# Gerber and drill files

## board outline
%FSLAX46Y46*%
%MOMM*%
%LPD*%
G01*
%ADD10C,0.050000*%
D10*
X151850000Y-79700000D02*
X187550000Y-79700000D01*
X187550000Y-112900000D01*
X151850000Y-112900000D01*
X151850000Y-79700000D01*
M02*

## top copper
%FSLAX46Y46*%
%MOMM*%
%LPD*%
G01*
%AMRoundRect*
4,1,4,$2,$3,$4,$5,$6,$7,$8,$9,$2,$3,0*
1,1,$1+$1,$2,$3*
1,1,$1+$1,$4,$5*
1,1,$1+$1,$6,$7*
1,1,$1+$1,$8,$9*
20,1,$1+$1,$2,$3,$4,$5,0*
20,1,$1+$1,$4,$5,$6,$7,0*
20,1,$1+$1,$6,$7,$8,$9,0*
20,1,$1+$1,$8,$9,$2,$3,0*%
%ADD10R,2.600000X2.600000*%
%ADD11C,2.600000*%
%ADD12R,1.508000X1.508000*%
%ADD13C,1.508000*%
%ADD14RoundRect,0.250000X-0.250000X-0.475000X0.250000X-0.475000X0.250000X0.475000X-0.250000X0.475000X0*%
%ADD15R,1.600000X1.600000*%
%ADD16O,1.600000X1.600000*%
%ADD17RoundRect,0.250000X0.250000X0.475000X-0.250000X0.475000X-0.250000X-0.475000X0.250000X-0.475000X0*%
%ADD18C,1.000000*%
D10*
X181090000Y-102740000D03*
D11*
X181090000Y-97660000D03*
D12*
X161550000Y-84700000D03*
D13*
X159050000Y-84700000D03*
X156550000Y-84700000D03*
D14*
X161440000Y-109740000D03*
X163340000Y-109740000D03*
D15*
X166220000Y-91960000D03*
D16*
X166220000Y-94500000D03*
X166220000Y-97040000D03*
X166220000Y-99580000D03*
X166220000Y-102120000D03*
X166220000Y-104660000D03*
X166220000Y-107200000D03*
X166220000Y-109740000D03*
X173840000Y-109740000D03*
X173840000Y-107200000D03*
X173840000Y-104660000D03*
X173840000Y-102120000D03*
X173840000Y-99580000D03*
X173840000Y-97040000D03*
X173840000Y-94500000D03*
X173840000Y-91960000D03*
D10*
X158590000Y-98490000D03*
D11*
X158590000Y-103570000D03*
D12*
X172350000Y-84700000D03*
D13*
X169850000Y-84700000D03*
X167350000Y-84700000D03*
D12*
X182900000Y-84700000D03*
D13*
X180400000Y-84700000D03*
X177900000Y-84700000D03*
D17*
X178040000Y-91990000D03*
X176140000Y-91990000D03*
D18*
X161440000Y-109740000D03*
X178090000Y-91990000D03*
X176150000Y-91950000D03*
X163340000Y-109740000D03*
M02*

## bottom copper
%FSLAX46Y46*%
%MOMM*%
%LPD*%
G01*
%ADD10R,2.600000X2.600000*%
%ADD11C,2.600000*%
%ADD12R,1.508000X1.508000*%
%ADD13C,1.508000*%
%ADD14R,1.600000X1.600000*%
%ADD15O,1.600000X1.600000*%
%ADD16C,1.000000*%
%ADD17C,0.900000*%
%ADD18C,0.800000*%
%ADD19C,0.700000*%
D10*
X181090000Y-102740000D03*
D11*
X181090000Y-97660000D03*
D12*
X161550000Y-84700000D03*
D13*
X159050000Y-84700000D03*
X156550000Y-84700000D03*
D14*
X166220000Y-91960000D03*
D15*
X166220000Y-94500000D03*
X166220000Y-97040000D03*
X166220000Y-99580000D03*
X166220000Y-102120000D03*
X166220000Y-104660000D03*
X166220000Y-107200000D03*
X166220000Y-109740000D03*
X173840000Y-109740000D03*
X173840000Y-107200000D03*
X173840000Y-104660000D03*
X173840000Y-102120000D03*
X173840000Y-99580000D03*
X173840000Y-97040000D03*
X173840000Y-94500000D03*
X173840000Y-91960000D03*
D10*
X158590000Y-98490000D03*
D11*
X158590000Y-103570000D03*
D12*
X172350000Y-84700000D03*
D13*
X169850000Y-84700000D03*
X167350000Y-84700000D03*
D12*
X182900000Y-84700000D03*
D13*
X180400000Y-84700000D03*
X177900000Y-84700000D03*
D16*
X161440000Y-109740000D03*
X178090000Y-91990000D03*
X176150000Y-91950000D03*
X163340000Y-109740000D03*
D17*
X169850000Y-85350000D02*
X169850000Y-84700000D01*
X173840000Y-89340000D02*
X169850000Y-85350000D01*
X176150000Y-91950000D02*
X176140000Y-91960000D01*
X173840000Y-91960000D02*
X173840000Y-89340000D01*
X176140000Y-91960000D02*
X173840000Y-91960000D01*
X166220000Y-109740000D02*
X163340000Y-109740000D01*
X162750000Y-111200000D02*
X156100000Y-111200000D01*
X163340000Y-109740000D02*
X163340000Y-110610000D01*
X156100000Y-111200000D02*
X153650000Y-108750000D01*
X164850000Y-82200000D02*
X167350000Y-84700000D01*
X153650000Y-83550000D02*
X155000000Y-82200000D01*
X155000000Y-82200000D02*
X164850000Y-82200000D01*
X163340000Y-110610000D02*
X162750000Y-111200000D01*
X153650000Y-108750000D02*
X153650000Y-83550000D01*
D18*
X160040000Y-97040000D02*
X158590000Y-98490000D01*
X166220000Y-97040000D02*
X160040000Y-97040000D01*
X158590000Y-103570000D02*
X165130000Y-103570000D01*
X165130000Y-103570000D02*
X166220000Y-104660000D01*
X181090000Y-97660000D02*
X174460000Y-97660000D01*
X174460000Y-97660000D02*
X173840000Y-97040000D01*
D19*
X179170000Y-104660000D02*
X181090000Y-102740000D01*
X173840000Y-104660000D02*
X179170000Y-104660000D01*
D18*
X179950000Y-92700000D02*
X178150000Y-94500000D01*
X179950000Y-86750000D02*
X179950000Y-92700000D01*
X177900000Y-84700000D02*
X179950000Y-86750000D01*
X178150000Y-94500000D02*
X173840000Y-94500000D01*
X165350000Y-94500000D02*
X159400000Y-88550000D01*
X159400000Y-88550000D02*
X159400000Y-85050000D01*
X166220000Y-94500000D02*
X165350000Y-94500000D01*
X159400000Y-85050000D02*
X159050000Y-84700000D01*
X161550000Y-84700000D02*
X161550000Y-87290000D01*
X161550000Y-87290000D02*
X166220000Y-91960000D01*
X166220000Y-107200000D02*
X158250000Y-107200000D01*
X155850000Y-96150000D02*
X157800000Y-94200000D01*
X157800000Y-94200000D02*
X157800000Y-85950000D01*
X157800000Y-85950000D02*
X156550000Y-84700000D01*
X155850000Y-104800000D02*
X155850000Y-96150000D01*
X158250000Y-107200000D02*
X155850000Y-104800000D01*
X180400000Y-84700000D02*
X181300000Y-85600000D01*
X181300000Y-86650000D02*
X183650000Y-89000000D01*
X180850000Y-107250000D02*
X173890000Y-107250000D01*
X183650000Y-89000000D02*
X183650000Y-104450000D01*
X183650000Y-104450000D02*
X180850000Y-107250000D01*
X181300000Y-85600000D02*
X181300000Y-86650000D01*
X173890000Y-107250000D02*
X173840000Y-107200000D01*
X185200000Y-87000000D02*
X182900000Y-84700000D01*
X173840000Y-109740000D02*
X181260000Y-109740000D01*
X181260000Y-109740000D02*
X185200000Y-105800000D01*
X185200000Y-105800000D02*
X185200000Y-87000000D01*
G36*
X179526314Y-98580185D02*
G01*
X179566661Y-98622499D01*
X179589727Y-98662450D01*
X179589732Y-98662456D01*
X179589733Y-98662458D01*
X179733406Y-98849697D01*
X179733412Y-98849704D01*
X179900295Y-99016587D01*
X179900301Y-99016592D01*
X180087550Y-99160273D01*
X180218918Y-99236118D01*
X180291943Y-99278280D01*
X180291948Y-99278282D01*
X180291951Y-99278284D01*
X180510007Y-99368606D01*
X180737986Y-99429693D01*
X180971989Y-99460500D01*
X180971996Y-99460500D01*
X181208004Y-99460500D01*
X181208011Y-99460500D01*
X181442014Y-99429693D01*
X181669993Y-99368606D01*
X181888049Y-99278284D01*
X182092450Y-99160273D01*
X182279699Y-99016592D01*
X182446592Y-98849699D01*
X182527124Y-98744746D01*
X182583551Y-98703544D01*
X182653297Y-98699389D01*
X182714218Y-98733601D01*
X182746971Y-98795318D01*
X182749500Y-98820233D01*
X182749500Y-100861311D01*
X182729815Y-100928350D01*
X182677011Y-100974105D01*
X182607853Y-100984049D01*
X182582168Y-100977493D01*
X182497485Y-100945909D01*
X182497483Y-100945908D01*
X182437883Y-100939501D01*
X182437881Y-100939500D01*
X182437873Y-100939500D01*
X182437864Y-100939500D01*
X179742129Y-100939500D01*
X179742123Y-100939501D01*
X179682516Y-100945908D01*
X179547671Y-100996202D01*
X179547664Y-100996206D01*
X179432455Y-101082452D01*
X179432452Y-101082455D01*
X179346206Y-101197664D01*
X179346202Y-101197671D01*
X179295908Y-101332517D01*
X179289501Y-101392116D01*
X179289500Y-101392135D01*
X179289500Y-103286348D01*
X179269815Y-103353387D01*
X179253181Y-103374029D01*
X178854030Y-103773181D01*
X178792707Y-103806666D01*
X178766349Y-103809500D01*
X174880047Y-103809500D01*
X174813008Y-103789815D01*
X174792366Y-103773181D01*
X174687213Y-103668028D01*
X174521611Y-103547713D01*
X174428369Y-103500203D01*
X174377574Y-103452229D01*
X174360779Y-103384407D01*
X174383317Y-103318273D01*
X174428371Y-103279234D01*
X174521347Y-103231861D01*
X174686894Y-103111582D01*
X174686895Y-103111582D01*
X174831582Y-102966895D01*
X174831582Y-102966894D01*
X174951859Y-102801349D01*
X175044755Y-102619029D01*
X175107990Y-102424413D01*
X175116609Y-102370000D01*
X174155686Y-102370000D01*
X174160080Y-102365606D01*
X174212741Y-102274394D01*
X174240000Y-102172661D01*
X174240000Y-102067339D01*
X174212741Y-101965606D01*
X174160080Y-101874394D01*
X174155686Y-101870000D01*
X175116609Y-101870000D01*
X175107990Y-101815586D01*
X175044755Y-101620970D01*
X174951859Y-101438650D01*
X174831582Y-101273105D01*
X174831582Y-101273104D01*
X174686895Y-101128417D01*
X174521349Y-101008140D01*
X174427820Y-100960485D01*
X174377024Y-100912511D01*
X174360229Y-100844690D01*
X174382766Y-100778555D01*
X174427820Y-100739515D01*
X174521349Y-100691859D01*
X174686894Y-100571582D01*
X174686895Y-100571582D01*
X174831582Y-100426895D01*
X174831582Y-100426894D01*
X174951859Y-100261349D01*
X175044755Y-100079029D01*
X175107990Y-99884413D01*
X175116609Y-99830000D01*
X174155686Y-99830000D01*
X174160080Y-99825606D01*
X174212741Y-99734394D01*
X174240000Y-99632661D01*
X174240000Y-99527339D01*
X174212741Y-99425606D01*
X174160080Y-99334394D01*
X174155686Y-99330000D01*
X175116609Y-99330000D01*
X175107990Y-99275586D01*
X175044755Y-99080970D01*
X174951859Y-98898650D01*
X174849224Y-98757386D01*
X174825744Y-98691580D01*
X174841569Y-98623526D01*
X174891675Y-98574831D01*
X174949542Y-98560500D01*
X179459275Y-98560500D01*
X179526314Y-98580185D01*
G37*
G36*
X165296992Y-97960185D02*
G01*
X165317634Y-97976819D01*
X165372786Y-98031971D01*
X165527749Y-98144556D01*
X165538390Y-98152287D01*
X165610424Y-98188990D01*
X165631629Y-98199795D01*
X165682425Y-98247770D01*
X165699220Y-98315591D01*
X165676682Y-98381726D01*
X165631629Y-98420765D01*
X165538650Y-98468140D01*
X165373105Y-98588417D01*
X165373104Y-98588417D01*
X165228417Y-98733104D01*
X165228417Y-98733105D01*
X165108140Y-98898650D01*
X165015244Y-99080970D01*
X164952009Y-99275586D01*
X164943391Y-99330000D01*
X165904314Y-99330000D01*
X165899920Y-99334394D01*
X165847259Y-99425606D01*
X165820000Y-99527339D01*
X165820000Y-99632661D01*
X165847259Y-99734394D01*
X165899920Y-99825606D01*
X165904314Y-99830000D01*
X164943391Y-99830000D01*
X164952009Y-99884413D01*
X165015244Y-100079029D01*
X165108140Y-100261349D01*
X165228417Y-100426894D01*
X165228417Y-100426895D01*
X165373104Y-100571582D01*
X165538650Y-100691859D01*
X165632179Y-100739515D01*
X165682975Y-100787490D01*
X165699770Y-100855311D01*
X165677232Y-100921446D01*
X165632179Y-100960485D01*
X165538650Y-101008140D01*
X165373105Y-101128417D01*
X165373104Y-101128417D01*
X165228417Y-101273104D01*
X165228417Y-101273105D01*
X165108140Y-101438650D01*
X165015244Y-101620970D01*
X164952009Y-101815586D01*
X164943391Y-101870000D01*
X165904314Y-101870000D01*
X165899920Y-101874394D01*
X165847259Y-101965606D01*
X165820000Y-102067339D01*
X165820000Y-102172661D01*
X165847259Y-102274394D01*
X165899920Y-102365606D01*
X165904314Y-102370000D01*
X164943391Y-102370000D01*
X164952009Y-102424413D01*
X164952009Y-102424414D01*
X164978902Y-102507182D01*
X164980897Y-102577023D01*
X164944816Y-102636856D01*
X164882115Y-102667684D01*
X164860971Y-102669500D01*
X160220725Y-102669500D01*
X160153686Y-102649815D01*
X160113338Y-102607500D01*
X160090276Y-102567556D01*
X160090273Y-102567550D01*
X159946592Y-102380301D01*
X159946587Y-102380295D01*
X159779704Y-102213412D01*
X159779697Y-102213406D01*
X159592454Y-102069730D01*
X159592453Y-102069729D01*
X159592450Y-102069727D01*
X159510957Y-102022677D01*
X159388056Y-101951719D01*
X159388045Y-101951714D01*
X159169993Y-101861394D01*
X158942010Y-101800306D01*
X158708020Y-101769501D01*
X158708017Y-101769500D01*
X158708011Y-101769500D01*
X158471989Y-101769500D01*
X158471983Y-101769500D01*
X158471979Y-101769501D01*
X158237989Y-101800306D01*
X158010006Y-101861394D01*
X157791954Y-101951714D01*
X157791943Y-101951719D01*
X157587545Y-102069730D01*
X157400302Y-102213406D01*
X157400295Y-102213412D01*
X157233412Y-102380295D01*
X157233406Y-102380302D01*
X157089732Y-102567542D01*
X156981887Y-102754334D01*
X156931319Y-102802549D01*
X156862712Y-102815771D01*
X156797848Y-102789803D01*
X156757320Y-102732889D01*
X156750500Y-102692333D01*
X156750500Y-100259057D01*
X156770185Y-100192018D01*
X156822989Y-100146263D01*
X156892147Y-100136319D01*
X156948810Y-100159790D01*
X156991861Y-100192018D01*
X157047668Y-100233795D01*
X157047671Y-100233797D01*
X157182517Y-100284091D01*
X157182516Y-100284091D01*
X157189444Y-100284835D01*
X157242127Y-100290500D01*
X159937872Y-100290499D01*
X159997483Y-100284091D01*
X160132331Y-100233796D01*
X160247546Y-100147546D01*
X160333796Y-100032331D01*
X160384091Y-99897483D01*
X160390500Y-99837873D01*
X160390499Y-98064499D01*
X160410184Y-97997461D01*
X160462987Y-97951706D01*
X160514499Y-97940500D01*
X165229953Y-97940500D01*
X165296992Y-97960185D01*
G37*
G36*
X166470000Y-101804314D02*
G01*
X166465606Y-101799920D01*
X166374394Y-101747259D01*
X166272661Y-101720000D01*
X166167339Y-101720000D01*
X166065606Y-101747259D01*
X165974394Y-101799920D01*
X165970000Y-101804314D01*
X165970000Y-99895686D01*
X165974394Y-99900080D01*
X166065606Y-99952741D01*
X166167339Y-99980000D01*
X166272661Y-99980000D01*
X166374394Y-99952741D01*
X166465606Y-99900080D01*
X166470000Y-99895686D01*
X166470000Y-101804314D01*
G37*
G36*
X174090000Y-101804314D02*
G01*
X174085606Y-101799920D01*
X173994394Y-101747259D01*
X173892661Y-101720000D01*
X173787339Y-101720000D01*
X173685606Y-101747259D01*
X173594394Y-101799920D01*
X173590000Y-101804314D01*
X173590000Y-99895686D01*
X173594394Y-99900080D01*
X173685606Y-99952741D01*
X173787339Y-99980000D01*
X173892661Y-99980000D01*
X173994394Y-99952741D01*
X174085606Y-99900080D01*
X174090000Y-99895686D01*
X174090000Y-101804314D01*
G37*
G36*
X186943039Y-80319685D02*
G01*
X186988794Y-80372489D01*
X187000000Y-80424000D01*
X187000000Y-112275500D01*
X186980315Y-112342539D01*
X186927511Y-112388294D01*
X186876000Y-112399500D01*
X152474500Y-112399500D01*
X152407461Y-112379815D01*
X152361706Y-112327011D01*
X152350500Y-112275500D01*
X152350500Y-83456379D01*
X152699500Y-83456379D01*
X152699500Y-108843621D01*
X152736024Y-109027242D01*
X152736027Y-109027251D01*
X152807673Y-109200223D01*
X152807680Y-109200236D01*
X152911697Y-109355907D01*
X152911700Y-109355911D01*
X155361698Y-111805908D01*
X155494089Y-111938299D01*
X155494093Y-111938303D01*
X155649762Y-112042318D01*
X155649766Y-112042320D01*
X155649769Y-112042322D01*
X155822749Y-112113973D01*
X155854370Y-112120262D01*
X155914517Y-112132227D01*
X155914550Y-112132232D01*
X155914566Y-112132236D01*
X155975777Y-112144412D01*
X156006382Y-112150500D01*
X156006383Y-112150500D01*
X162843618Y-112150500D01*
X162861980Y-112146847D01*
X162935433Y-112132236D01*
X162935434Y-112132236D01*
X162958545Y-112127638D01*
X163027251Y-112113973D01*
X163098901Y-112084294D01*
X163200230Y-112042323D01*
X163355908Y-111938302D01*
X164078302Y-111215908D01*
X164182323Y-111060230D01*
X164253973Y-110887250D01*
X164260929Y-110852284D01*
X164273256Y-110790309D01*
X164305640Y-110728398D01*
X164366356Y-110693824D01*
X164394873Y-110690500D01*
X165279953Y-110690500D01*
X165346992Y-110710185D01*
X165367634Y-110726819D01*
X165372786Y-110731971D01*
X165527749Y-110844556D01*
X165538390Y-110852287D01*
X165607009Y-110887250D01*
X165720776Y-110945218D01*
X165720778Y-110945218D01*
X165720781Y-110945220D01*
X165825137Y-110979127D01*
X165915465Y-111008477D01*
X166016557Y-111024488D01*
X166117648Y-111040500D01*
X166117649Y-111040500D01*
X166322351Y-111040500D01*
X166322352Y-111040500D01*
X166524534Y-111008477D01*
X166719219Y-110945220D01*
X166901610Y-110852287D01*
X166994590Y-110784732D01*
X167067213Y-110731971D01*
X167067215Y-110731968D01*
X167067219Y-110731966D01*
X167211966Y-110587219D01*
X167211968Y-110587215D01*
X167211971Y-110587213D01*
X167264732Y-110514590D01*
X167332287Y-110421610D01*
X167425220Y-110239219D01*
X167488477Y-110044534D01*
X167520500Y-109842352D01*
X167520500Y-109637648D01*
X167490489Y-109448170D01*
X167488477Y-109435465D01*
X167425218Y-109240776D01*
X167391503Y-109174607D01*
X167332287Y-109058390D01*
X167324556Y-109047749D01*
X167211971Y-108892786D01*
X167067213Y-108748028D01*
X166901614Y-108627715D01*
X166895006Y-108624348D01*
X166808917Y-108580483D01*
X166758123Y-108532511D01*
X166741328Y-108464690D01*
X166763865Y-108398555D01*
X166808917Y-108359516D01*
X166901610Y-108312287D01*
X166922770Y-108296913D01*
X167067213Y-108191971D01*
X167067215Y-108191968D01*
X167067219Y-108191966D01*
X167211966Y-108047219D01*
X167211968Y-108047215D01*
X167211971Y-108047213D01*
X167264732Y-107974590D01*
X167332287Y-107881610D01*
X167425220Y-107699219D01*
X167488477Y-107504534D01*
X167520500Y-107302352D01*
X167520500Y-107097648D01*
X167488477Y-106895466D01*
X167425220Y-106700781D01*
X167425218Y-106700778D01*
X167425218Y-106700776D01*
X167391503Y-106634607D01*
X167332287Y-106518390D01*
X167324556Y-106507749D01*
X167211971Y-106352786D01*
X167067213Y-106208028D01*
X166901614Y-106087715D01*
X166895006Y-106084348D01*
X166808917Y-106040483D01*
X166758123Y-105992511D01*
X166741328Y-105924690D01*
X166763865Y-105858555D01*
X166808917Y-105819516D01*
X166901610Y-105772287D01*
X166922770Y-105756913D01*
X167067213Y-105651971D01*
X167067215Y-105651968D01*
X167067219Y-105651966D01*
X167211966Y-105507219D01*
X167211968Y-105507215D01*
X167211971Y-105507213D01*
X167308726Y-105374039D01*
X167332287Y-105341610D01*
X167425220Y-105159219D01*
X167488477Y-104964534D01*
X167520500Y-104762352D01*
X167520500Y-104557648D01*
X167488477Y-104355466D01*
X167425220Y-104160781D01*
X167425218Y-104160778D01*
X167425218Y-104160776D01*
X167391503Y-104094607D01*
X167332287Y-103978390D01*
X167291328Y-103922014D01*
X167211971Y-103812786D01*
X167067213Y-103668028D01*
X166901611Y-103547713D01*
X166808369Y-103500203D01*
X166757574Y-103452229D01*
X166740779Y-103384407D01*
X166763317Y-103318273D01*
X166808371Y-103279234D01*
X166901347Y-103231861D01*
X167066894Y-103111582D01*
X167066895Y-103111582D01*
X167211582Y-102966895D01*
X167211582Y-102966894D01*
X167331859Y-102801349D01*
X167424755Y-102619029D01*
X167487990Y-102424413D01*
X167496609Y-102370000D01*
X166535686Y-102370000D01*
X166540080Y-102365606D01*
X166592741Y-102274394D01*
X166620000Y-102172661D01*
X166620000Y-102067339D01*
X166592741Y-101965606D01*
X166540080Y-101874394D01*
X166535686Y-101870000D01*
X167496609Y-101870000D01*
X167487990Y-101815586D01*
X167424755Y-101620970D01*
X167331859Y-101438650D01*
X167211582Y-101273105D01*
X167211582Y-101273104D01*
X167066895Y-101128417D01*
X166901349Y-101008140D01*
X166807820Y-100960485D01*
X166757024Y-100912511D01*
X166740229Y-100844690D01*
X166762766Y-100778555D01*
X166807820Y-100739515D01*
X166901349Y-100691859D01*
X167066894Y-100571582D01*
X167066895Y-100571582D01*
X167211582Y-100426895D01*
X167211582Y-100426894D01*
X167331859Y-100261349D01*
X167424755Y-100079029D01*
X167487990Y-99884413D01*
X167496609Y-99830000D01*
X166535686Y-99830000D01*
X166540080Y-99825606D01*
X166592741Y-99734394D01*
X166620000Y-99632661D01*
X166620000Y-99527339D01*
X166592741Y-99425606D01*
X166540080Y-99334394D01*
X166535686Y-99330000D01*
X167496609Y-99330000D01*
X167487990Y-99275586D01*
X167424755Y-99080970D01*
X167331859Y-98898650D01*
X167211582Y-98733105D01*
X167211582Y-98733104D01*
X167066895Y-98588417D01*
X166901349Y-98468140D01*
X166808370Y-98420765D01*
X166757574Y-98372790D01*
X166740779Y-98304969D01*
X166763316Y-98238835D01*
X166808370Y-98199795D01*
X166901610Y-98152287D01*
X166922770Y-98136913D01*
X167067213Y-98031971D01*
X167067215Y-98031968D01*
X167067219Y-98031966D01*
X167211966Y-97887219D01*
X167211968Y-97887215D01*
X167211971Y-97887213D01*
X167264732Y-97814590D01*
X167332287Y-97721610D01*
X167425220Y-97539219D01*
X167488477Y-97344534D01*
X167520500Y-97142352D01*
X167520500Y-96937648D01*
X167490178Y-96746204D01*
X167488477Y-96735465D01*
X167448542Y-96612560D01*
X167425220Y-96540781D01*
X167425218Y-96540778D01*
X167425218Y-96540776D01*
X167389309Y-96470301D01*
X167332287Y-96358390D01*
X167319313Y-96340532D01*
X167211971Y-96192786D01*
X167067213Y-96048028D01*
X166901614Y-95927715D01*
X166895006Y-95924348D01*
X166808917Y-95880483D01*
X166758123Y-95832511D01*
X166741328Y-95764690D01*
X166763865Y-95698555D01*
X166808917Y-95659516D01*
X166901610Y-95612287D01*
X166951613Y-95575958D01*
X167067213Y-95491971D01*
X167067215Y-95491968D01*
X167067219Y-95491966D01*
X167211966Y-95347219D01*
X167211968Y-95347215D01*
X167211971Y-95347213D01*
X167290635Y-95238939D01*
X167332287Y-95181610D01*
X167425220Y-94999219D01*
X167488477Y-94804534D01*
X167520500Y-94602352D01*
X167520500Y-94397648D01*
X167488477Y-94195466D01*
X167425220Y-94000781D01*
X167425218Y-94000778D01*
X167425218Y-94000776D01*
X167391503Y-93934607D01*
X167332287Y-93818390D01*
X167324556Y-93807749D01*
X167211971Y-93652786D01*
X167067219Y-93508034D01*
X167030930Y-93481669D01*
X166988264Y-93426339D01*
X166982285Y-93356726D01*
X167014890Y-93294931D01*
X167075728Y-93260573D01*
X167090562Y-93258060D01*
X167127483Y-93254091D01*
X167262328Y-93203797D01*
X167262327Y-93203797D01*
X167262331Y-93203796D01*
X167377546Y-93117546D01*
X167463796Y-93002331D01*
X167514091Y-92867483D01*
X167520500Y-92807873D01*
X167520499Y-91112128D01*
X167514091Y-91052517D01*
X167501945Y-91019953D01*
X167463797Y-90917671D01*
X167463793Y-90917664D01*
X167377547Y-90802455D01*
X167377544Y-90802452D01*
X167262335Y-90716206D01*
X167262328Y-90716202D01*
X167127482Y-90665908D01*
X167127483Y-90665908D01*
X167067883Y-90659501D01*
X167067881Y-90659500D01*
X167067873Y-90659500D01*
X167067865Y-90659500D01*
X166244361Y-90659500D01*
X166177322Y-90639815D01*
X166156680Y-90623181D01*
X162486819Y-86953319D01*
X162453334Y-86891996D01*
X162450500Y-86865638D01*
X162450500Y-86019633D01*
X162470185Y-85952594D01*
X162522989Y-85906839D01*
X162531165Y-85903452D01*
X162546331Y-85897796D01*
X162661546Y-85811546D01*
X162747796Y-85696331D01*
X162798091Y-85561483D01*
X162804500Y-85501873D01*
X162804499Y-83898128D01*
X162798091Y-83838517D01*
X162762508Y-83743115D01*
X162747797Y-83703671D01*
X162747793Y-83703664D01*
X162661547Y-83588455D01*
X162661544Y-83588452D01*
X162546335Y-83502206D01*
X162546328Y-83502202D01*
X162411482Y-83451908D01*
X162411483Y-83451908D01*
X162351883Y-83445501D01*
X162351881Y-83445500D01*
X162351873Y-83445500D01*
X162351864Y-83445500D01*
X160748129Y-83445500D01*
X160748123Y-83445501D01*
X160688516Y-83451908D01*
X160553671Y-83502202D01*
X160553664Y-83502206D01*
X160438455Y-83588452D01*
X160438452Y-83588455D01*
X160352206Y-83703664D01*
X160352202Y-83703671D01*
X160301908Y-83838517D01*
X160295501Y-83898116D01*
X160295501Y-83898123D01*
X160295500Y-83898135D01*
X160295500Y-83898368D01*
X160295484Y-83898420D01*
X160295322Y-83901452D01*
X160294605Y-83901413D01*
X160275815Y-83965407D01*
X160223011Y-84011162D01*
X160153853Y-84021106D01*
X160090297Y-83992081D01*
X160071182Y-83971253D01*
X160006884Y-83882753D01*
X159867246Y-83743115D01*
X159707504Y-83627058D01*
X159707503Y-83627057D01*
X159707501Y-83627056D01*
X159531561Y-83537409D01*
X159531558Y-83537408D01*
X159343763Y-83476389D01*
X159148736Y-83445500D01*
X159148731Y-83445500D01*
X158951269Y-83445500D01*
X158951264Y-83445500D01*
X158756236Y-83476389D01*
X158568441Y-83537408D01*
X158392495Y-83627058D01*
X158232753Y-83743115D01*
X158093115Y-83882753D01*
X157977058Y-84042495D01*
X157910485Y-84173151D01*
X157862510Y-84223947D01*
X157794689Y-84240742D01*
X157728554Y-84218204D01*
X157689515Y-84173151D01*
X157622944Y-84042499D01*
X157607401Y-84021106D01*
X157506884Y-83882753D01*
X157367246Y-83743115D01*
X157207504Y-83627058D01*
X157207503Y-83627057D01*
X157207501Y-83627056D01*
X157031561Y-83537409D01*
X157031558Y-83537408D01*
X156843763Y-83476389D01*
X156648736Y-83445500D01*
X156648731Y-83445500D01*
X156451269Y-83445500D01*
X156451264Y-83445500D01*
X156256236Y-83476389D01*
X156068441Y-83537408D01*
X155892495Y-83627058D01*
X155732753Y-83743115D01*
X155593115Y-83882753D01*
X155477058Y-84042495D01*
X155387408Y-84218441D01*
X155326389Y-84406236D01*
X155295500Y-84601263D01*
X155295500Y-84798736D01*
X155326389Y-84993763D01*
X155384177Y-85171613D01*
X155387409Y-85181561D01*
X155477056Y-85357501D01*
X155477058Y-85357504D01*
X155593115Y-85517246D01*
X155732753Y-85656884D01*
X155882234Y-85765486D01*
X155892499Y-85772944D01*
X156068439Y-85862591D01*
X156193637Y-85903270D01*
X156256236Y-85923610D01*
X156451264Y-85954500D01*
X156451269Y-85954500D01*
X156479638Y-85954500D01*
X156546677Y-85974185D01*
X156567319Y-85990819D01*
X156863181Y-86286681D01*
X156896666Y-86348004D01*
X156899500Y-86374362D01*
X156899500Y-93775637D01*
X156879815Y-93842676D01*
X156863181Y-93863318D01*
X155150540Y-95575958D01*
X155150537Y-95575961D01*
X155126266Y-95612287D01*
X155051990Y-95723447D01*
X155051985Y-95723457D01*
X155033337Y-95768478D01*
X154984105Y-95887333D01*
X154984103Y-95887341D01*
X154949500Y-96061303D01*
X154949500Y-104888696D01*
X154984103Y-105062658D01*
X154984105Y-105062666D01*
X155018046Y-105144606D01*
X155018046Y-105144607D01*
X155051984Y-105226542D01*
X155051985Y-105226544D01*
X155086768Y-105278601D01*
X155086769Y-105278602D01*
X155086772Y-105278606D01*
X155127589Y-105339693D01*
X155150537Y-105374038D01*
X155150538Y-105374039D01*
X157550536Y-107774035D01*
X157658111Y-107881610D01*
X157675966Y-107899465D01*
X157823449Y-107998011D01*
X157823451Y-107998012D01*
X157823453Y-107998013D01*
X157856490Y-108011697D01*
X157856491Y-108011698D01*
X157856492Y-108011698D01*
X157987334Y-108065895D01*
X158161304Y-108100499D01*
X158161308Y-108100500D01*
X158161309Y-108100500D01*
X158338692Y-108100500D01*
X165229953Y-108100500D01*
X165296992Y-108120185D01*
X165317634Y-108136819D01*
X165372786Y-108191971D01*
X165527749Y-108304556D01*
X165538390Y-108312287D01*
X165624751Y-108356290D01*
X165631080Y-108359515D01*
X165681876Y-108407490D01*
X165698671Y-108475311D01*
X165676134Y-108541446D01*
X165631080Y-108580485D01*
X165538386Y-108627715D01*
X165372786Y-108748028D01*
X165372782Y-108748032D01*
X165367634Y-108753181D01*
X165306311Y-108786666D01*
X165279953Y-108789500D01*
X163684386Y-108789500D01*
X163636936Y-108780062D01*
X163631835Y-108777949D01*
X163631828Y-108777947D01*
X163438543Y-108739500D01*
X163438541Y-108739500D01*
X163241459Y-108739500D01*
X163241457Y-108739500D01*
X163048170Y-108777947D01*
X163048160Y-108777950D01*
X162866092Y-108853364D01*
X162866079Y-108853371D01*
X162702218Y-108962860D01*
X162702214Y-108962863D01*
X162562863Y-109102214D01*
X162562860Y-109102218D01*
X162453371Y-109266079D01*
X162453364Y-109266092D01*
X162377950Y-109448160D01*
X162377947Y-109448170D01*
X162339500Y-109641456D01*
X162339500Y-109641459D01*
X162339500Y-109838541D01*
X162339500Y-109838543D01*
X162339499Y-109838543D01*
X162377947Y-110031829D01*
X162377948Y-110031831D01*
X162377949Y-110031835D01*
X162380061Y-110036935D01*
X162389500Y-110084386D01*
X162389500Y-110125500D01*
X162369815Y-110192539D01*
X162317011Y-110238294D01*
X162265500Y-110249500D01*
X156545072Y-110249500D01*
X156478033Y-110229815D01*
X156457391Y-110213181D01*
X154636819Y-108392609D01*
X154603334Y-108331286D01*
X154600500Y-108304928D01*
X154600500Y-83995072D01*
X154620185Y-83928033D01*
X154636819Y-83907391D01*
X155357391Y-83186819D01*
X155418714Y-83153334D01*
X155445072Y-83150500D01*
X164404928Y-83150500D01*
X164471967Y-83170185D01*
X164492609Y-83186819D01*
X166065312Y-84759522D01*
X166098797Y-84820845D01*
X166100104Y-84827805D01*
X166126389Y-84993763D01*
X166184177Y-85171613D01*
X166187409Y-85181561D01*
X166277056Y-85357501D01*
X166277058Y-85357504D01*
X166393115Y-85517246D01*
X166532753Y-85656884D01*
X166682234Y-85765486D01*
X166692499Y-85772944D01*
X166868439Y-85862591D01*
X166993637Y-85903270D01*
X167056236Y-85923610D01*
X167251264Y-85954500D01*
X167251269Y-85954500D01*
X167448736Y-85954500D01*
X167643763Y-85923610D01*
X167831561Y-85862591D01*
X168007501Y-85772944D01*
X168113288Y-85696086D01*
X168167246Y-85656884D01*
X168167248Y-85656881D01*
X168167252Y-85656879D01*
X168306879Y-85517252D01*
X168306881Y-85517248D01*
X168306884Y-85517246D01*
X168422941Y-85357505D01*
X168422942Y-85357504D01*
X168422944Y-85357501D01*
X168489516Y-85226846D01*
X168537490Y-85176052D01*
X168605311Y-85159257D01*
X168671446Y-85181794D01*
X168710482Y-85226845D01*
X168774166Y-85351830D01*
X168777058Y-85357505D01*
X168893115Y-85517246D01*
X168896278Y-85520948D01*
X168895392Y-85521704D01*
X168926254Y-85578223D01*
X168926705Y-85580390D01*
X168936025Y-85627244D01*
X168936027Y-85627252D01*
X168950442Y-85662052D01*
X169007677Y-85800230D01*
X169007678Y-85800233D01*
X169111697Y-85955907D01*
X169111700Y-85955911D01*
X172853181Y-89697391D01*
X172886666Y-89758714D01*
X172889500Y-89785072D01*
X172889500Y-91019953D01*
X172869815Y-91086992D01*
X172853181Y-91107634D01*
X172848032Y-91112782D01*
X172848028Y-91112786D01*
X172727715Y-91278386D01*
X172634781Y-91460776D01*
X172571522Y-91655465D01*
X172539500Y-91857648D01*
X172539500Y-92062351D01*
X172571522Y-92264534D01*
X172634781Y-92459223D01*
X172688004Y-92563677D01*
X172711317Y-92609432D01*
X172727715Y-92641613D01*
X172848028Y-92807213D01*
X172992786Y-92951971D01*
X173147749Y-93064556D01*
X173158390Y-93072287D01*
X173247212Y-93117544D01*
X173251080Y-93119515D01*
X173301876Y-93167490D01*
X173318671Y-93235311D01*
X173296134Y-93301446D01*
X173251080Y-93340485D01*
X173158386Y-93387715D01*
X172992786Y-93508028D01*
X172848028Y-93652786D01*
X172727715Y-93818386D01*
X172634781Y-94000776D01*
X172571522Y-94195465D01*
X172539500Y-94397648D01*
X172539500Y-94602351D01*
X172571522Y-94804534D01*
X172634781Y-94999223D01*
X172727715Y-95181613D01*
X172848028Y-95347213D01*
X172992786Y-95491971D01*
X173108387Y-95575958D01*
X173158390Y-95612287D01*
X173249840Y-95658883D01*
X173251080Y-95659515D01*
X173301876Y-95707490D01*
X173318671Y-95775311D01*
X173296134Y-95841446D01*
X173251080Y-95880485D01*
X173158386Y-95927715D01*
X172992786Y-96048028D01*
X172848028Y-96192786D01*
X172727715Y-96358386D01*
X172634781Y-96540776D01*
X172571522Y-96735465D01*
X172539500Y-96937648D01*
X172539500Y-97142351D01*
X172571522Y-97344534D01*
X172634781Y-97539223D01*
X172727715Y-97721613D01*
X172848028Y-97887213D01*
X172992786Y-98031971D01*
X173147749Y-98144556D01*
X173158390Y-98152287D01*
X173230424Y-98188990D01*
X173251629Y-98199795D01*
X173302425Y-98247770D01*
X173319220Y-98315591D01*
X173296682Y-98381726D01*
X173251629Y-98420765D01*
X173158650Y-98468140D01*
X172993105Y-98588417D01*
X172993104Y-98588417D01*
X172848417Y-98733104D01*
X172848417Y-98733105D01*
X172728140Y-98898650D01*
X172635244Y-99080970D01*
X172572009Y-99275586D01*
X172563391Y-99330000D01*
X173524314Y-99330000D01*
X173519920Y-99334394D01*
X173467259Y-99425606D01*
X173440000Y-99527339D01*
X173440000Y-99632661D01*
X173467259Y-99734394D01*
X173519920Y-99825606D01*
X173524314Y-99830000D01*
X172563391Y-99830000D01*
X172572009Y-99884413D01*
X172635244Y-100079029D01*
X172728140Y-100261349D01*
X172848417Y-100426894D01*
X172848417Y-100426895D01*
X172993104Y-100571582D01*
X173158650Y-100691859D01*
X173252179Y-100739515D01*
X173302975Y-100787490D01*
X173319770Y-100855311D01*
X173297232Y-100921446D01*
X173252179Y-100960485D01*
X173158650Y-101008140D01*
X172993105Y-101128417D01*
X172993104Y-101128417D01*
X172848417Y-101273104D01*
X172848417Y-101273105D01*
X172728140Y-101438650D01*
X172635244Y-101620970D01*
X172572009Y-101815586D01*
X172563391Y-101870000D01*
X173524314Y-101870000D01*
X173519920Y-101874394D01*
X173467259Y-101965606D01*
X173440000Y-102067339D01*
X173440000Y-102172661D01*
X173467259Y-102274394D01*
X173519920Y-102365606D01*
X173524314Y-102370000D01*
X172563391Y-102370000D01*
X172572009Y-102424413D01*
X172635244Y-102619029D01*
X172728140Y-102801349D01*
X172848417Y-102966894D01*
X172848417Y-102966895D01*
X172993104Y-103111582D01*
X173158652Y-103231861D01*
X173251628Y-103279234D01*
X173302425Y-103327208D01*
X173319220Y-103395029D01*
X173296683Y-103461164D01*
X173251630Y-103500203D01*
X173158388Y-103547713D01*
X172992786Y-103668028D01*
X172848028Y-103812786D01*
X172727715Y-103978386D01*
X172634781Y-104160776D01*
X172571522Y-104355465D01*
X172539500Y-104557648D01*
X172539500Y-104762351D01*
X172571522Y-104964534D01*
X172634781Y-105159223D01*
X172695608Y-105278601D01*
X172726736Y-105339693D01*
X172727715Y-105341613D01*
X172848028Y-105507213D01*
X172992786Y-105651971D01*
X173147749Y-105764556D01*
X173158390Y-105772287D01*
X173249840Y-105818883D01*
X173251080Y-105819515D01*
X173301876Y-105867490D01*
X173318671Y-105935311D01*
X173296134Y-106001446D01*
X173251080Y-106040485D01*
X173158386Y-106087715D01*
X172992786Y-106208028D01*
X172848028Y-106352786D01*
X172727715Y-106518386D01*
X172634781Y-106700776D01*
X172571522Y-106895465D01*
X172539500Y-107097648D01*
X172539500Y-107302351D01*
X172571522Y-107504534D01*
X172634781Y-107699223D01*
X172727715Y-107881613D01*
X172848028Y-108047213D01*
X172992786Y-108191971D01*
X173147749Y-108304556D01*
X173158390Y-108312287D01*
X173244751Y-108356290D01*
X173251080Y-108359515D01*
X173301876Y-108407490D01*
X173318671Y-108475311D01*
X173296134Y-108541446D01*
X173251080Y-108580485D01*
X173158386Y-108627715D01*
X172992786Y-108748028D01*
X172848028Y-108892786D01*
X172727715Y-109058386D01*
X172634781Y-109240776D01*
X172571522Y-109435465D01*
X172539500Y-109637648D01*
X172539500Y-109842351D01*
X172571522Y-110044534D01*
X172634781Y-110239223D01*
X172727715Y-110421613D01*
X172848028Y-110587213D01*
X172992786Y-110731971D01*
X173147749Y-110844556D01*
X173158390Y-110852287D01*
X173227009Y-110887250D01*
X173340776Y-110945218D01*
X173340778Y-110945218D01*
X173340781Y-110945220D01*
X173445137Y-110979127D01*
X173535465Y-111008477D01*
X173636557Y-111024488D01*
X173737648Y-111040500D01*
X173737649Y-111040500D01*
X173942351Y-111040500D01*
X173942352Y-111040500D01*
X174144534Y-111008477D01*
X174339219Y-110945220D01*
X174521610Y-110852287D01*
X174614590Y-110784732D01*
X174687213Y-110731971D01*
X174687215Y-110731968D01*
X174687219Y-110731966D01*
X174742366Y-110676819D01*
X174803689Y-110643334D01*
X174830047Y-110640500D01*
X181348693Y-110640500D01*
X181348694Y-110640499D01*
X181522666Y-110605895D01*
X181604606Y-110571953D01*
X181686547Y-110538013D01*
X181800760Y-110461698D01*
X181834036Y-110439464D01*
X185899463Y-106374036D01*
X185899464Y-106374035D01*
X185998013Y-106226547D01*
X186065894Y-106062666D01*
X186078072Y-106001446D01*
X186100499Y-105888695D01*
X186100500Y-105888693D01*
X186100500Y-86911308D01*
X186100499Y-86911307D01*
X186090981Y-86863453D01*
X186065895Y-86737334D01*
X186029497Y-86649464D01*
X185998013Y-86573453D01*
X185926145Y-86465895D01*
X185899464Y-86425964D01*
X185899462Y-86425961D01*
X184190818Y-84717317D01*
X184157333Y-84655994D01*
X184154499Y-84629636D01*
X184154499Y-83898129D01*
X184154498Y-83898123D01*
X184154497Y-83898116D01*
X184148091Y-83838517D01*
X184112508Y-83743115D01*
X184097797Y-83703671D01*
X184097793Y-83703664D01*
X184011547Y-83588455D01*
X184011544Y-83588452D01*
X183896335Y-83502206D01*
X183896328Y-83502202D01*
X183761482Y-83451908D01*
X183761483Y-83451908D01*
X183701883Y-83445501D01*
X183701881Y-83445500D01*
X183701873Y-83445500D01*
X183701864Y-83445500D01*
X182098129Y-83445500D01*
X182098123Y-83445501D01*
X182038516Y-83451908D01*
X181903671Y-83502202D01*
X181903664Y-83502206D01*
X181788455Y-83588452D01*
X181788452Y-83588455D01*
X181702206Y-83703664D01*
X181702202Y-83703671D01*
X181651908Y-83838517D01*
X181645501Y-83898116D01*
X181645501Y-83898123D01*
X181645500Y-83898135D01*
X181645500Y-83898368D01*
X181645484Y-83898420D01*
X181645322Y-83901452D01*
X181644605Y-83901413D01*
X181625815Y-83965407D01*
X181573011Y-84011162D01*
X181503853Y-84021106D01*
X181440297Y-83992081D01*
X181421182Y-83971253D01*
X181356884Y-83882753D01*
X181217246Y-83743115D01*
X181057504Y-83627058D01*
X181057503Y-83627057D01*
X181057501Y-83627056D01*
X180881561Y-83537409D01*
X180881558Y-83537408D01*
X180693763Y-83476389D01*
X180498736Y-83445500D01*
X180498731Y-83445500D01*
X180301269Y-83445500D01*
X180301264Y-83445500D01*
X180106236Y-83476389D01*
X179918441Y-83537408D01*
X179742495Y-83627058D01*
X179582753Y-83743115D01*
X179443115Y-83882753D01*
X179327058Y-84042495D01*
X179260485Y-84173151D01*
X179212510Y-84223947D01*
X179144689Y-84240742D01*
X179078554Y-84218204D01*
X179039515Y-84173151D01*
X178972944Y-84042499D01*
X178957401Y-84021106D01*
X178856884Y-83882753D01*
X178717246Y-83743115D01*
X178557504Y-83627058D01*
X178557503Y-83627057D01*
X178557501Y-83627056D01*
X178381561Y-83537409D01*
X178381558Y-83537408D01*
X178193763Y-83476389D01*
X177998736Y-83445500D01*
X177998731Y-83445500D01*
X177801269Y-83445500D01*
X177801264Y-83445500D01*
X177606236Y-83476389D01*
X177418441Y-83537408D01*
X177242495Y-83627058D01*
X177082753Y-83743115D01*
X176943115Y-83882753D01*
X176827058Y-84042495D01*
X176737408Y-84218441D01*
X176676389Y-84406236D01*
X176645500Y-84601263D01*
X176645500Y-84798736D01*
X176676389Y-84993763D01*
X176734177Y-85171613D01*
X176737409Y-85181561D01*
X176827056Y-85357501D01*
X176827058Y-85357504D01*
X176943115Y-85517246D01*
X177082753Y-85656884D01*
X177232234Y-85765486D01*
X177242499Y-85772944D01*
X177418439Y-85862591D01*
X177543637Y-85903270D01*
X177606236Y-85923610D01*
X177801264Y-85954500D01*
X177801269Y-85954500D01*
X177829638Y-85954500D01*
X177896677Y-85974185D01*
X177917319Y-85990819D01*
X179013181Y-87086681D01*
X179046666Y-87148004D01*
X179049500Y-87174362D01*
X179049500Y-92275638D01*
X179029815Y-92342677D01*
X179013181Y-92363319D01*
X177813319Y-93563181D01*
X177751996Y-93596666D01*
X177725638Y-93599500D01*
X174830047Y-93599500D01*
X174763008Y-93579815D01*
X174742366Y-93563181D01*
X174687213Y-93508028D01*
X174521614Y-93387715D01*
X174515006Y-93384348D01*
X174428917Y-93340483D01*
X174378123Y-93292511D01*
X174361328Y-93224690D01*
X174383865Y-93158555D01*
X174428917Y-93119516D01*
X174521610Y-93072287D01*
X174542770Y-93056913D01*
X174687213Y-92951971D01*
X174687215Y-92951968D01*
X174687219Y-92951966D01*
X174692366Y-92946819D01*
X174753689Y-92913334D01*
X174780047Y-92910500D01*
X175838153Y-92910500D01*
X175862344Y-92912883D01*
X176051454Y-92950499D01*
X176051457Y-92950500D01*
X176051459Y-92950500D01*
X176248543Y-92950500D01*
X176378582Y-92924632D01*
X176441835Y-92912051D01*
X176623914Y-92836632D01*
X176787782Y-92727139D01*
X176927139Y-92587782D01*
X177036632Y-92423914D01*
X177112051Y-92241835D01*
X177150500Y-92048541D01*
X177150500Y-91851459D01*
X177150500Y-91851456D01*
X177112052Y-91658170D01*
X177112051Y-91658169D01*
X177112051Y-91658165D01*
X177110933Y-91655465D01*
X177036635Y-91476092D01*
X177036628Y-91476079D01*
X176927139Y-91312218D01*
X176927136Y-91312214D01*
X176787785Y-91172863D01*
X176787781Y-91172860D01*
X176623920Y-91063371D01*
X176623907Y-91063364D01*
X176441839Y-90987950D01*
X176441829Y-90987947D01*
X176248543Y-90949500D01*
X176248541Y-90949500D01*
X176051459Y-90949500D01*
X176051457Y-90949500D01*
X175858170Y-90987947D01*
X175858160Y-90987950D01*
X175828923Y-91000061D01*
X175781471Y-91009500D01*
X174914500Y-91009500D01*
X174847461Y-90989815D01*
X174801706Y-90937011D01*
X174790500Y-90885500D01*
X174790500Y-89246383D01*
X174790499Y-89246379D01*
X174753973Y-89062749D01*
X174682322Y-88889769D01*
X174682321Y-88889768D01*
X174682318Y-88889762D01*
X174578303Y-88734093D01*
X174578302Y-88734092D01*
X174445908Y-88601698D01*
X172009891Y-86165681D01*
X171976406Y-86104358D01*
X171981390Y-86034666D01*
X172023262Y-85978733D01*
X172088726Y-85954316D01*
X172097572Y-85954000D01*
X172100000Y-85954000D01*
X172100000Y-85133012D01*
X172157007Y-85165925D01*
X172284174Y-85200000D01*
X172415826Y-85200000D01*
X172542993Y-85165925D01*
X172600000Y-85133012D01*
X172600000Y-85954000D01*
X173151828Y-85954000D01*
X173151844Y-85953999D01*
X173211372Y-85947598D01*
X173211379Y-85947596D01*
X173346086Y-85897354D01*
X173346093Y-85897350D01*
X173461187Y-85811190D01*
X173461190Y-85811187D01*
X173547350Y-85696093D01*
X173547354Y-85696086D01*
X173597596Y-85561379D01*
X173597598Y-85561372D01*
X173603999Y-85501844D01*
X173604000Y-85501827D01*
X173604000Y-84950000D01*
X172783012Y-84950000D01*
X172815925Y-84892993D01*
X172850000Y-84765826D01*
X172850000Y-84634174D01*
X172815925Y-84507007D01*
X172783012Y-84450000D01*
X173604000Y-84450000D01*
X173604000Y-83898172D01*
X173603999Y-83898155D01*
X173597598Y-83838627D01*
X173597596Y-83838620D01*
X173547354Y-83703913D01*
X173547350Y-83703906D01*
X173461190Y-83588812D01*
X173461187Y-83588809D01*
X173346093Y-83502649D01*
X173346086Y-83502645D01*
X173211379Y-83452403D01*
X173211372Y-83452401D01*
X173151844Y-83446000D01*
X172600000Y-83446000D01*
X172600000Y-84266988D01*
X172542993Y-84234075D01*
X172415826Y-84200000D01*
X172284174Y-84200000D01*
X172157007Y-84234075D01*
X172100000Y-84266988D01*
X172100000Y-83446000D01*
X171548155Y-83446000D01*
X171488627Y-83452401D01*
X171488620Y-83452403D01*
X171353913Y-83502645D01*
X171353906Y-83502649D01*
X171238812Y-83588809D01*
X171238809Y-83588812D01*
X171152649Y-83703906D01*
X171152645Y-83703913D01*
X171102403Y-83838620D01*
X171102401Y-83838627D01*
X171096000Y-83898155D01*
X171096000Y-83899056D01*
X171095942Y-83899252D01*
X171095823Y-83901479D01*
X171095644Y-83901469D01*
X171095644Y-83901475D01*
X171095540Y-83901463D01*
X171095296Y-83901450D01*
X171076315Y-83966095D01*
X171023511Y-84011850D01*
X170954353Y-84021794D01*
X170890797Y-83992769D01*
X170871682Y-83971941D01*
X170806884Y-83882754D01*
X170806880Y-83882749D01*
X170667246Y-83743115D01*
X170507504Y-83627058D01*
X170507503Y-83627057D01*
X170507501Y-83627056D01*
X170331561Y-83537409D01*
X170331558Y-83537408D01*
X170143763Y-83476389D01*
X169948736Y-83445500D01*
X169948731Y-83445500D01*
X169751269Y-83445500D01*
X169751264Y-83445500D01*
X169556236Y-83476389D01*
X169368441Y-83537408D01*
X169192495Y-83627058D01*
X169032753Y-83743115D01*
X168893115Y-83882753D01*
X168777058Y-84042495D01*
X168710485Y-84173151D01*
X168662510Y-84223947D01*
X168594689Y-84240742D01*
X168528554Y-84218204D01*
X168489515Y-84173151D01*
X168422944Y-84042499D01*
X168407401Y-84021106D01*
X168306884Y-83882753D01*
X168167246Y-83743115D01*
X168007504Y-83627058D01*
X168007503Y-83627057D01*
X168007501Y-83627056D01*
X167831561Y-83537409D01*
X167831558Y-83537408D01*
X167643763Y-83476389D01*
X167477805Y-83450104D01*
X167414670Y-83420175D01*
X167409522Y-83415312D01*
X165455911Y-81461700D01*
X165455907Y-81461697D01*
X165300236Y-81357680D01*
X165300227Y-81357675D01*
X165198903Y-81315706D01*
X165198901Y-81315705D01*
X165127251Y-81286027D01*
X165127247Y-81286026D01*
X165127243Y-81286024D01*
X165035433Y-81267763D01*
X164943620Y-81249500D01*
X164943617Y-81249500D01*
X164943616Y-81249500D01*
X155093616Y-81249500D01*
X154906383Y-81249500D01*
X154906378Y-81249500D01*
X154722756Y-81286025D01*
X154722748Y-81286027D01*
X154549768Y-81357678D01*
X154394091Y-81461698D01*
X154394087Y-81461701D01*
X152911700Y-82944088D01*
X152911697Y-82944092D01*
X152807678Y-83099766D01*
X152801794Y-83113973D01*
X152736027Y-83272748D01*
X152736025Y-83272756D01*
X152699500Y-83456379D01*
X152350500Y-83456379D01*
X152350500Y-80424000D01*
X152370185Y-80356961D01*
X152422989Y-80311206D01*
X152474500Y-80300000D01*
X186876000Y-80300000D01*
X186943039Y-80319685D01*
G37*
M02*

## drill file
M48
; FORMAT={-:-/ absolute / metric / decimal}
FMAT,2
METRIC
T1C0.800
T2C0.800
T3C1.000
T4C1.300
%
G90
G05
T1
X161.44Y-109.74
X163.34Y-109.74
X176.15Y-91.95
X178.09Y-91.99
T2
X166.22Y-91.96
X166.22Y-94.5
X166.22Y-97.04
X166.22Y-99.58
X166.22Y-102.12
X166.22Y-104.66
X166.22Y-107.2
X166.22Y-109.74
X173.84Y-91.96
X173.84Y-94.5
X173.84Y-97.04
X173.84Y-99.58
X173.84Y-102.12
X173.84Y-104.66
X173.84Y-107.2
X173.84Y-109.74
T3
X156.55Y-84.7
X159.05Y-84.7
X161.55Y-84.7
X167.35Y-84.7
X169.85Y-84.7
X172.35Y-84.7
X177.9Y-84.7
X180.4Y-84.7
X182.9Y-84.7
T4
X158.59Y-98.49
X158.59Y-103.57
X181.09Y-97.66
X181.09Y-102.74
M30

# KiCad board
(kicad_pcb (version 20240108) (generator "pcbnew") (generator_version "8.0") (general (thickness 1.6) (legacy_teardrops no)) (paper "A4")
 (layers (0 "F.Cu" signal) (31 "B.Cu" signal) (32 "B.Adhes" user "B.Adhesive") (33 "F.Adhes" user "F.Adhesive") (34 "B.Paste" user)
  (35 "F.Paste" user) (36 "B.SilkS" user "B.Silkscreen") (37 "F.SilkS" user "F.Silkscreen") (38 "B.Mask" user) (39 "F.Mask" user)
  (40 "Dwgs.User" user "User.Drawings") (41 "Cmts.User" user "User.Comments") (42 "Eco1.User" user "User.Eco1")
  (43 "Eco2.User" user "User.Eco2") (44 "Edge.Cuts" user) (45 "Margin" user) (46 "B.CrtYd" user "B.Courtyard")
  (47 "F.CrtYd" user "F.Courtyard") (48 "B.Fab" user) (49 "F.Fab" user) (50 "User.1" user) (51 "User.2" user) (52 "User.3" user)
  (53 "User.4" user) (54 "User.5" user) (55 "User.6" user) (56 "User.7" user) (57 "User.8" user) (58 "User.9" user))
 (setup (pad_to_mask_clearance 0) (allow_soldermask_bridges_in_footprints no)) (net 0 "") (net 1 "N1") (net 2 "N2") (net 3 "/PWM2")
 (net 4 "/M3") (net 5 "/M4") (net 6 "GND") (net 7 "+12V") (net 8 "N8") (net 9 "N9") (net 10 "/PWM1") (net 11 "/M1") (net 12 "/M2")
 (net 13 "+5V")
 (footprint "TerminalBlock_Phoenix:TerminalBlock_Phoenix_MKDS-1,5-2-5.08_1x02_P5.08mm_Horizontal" (layer "F.Cu") (at 181.09 102.74 90)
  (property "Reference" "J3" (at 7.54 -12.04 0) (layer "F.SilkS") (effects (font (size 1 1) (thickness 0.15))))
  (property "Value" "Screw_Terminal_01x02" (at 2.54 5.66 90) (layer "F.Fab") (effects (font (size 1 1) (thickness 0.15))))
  (pad "1" thru_hole rect (at 0 0 90) (size 2.6 2.6) (drill 1.3) (layers "*.Cu" "*.Mask") (remove_unused_layers no) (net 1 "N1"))
  (pad "2" thru_hole circle (at 5.08 0 90) (size 2.6 2.6) (drill 1.3) (layers "*.Cu" "*.Mask") (remove_unused_layers no) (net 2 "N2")))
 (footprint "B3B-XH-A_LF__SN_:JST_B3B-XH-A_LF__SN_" (layer "F.Cu") (at 159.05 84.175)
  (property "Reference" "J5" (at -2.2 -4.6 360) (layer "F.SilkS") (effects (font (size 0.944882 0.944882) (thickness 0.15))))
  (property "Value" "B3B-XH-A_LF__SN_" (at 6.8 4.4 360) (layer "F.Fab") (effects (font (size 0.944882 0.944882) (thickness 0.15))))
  (pad "1" thru_hole rect (at 2.5 0.525) (size 1.508 1.508) (drill 1) (layers "*.Cu" "*.Mask") (remove_unused_layers no) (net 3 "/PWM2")
   (solder_mask_margin 0.102))
  (pad "2" thru_hole circle (at 0 0.525) (size 1.508 1.508) (drill 1) (layers "*.Cu" "*.Mask") (remove_unused_layers no) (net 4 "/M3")
   (solder_mask_margin 0.102))
  (pad "3" thru_hole circle (at -2.5 0.525) (size 1.508 1.508) (drill 1) (layers "*.Cu" "*.Mask") (remove_unused_layers no) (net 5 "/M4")
   (solder_mask_margin 0.102)))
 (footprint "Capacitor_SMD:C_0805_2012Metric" (layer "F.Cu") (at 162.39 109.74)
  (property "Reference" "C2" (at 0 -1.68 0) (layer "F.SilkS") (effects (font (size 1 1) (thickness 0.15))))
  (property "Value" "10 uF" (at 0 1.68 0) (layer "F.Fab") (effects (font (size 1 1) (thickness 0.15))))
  (pad "1" smd roundrect (at -0.95 0) (size 1 1.45) (layers "F.Cu" "F.Paste" "F.Mask") (roundrect_rratio 0.25) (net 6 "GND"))
  (pad "2" smd roundrect (at 0.95 0) (size 1 1.45) (layers "F.Cu" "F.Paste" "F.Mask") (roundrect_rratio 0.25) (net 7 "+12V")))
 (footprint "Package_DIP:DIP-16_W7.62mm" (layer "F.Cu") (at 166.22 91.96)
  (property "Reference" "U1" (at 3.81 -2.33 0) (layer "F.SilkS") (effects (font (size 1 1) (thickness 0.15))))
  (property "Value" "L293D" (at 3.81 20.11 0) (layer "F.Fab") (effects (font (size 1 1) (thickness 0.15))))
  (pad "1" thru_hole rect (at 0 0) (size 1.6 1.6) (drill 0.8) (layers "*.Cu" "*.Mask") (remove_unused_layers no) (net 3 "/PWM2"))
  (pad "2" thru_hole oval (at 0 2.54) (size 1.6 1.6) (drill 0.8) (layers "*.Cu" "*.Mask") (remove_unused_layers no) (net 4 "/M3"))
  (pad "3" thru_hole oval (at 0 5.08) (size 1.6 1.6) (drill 0.8) (layers "*.Cu" "*.Mask") (remove_unused_layers no) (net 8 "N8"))
  (pad "4" thru_hole oval (at 0 7.62) (size 1.6 1.6) (drill 0.8) (layers "*.Cu" "*.Mask") (remove_unused_layers no) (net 6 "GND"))
  (pad "5" thru_hole oval (at 0 10.16) (size 1.6 1.6) (drill 0.8) (layers "*.Cu" "*.Mask") (remove_unused_layers no) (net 6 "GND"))
  (pad "6" thru_hole oval (at 0 12.7) (size 1.6 1.6) (drill 0.8) (layers "*.Cu" "*.Mask") (remove_unused_layers no) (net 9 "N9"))
  (pad "7" thru_hole oval (at 0 15.24) (size 1.6 1.6) (drill 0.8) (layers "*.Cu" "*.Mask") (remove_unused_layers no) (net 5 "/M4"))
  (pad "8" thru_hole oval (at 0 17.78) (size 1.6 1.6) (drill 0.8) (layers "*.Cu" "*.Mask") (remove_unused_layers no) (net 7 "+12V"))
  (pad "9" thru_hole oval (at 7.62 17.78) (size 1.6 1.6) (drill 0.8) (layers "*.Cu" "*.Mask") (remove_unused_layers no) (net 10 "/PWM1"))
  (pad "10" thru_hole oval (at 7.62 15.24) (size 1.6 1.6) (drill 0.8) (layers "*.Cu" "*.Mask") (remove_unused_layers no) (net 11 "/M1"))
  (pad "11" thru_hole oval (at 7.62 12.7) (size 1.6 1.6) (drill 0.8) (layers "*.Cu" "*.Mask") (remove_unused_layers no) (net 1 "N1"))
  (pad "12" thru_hole oval (at 7.62 10.16) (size 1.6 1.6) (drill 0.8) (layers "*.Cu" "*.Mask") (remove_unused_layers no) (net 6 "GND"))
  (pad "13" thru_hole oval (at 7.62 7.62) (size 1.6 1.6) (drill 0.8) (layers "*.Cu" "*.Mask") (remove_unused_layers no) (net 6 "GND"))
  (pad "14" thru_hole oval (at 7.62 5.08) (size 1.6 1.6) (drill 0.8) (layers "*.Cu" "*.Mask") (remove_unused_layers no) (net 2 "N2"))
  (pad "15" thru_hole oval (at 7.62 2.54) (size 1.6 1.6) (drill 0.8) (layers "*.Cu" "*.Mask") (remove_unused_layers no) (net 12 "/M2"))
  (pad "16" thru_hole oval (at 7.62 0) (size 1.6 1.6) (drill 0.8) (layers "*.Cu" "*.Mask") (remove_unused_layers no) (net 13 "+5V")))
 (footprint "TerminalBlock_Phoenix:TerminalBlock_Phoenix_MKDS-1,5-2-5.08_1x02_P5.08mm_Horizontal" (layer "F.Cu") (at 158.59 98.49 -90)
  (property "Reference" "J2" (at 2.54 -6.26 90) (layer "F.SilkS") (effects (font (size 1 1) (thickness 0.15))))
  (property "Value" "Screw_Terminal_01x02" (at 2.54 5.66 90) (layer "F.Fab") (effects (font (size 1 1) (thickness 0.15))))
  (pad "1" thru_hole rect (at 0 0 270) (size 2.6 2.6) (drill 1.3) (layers "*.Cu" "*.Mask") (remove_unused_layers no) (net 8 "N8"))
  (pad "2" thru_hole circle (at 5.08 0 270) (size 2.6 2.6) (drill 1.3) (layers "*.Cu" "*.Mask") (remove_unused_layers no) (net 9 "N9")))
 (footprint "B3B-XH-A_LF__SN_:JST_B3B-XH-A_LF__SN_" (layer "F.Cu") (at 169.85 84.175)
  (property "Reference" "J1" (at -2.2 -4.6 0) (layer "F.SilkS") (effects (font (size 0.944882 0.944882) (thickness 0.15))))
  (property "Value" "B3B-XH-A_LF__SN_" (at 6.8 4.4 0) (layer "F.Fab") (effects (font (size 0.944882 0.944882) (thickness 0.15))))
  (pad "1" thru_hole rect (at 2.5 0.525) (size 1.508 1.508) (drill 1) (layers "*.Cu" "*.Mask") (remove_unused_layers no) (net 6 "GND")
   (solder_mask_margin 0.102))
  (pad "2" thru_hole circle (at 0 0.525) (size 1.508 1.508) (drill 1) (layers "*.Cu" "*.Mask") (remove_unused_layers no) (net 13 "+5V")
   (solder_mask_margin 0.102))
  (pad "3" thru_hole circle (at -2.5 0.525) (size 1.508 1.508) (drill 1) (layers "*.Cu" "*.Mask") (remove_unused_layers no) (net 7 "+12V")
   (solder_mask_margin 0.102)))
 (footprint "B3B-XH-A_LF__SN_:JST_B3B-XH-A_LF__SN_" (layer "F.Cu") (at 180.4 84.175)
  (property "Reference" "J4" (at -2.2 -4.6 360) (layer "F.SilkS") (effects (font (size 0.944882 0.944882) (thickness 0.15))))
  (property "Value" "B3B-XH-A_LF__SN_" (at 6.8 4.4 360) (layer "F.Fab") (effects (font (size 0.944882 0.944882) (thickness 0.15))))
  (pad "1" thru_hole rect (at 2.5 0.525) (size 1.508 1.508) (drill 1) (layers "*.Cu" "*.Mask") (remove_unused_layers no) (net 10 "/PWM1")
   (solder_mask_margin 0.102))
  (pad "2" thru_hole circle (at 0 0.525) (size 1.508 1.508) (drill 1) (layers "*.Cu" "*.Mask") (remove_unused_layers no) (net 11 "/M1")
   (solder_mask_margin 0.102))
  (pad "3" thru_hole circle (at -2.5 0.525) (size 1.508 1.508) (drill 1) (layers "*.Cu" "*.Mask") (remove_unused_layers no) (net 12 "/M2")
   (solder_mask_margin 0.102)))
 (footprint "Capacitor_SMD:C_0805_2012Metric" (layer "F.Cu") (at 177.09 91.99 180)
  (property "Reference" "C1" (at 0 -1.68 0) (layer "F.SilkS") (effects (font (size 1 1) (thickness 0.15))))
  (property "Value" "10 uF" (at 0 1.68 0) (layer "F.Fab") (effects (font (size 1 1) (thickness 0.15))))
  (pad "1" smd roundrect (at -0.95 0 180) (size 1 1.45) (layers "F.Cu" "F.Paste" "F.Mask") (roundrect_rratio 0.25) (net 6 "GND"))
  (pad "2" smd roundrect (at 0.95 0 180) (size 1 1.45) (layers "F.Cu" "F.Paste" "F.Mask") (roundrect_rratio 0.25) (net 13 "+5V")))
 (gr_rect (start 151.85 79.7) (end 187.55 112.9) (stroke (width 0.05) (type default)) (fill none) (layer "Edge.Cuts"))
 (via (at 161.44 109.74) (size 1) (drill 0.8) (layers "F.Cu" "B.Cu") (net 6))
 (via (at 178.09 91.99) (size 1) (drill 0.8) (layers "F.Cu" "B.Cu") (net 6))
 (via (at 176.15 91.95) (size 1) (drill 0.8) (layers "F.Cu" "B.Cu") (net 13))
 (segment (start 169.85 85.35) (end 169.85 84.7) (width 0.9) (layer "B.Cu") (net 13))
 (segment (start 173.84 89.34) (end 169.85 85.35) (width 0.9) (layer "B.Cu") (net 13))
 (segment (start 176.15 91.95) (end 176.14 91.96) (width 0.9) (layer "B.Cu") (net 13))
 (segment (start 173.84 91.96) (end 173.84 89.34) (width 0.9) (layer "B.Cu") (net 13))
 (segment (start 176.14 91.96) (end 173.84 91.96) (width 0.9) (layer "B.Cu") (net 13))
 (via (at 163.34 109.74) (size 1) (drill 0.8) (layers "F.Cu" "B.Cu") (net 7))
 (segment (start 166.22 109.74) (end 163.34 109.74) (width 0.9) (layer "B.Cu") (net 7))
 (segment (start 162.75 111.2) (end 156.1 111.2) (width 0.9) (layer "B.Cu") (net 7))
 (segment (start 163.34 109.74) (end 163.34 110.61) (width 0.9) (layer "B.Cu") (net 7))
 (segment (start 156.1 111.2) (end 153.65 108.75) (width 0.9) (layer "B.Cu") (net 7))
 (segment (start 164.85 82.2) (end 167.35 84.7) (width 0.9) (layer "B.Cu") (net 7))
 (segment (start 153.65 83.55) (end 155 82.2) (width 0.9) (layer "B.Cu") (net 7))
 (segment (start 155 82.2) (end 164.85 82.2) (width 0.9) (layer "B.Cu") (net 7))
 (segment (start 163.34 110.61) (end 162.75 111.2) (width 0.9) (layer "B.Cu") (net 7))
 (segment (start 153.65 108.75) (end 153.65 83.55) (width 0.9) (layer "B.Cu") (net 7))
 (segment (start 160.04 97.04) (end 158.59 98.49) (width 0.8) (layer "B.Cu") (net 8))
 (segment (start 166.22 97.04) (end 160.04 97.04) (width 0.8) (layer "B.Cu") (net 8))
 (segment (start 158.59 103.57) (end 165.13 103.57) (width 0.8) (layer "B.Cu") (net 9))
 (segment (start 165.13 103.57) (end 166.22 104.66) (width 0.8) (layer "B.Cu") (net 9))
 (segment (start 181.09 97.66) (end 174.46 97.66) (width 0.8) (layer "B.Cu") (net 2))
 (segment (start 174.46 97.66) (end 173.84 97.04) (width 0.8) (layer "B.Cu") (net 2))
 (segment (start 179.17 104.66) (end 181.09 102.74) (width 0.7) (layer "B.Cu") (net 1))
 (segment (start 173.84 104.66) (end 179.17 104.66) (width 0.7) (layer "B.Cu") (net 1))
 (segment (start 179.95 92.7) (end 178.15 94.5) (width 0.8) (layer "B.Cu") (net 12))
 (segment (start 179.95 86.75) (end 179.95 92.7) (width 0.8) (layer "B.Cu") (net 12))
 (segment (start 177.9 84.7) (end 179.95 86.75) (width 0.8) (layer "B.Cu") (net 12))
 (segment (start 178.15 94.5) (end 173.84 94.5) (width 0.8) (layer "B.Cu") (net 12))
 (segment (start 165.35 94.5) (end 159.4 88.55) (width 0.8) (layer "B.Cu") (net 4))
 (segment (start 159.4 88.55) (end 159.4 85.05) (width 0.8) (layer "B.Cu") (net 4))
 (segment (start 166.22 94.5) (end 165.35 94.5) (width 0.8) (layer "B.Cu") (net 4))
 (segment (start 159.4 85.05) (end 159.05 84.7) (width 0.8) (layer "B.Cu") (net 4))
 (segment (start 161.55 84.7) (end 161.55 87.29) (width 0.8) (layer "B.Cu") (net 3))
 (segment (start 161.55 87.29) (end 166.22 91.96) (width 0.8) (layer "B.Cu") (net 3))
 (segment (start 166.22 107.2) (end 158.25 107.2) (width 0.8) (layer "B.Cu") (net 5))
 (segment (start 155.85 96.15) (end 157.8 94.2) (width 0.8) (layer "B.Cu") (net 5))
 (segment (start 157.8 94.2) (end 157.8 85.95) (width 0.8) (layer "B.Cu") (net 5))
 (segment (start 157.8 85.95) (end 156.55 84.7) (width 0.8) (layer "B.Cu") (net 5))
 (segment (start 155.85 104.8) (end 155.85 96.15) (width 0.8) (layer "B.Cu") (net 5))
 (segment (start 158.25 107.2) (end 155.85 104.8) (width 0.8) (layer "B.Cu") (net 5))
 (segment (start 180.4 84.7) (end 181.3 85.6) (width 0.8) (layer "B.Cu") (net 11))
 (segment (start 181.3 86.65) (end 183.65 89) (width 0.8) (layer "B.Cu") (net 11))
 (segment (start 180.85 107.25) (end 173.89 107.25) (width 0.8) (layer "B.Cu") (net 11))
 (segment (start 183.65 89) (end 183.65 104.45) (width 0.8) (layer "B.Cu") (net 11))
 (segment (start 183.65 104.45) (end 180.85 107.25) (width 0.8) (layer "B.Cu") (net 11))
 (segment (start 181.3 85.6) (end 181.3 86.65) (width 0.8) (layer "B.Cu") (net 11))
 (segment (start 173.89 107.25) (end 173.84 107.2) (width 0.8) (layer "B.Cu") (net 11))
 (segment (start 185.2 87) (end 182.9 84.7) (width 0.8) (layer "B.Cu") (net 10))
 (segment (start 173.84 109.74) (end 181.26 109.74) (width 0.8) (layer "B.Cu") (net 10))
 (segment (start 181.26 109.74) (end 185.2 105.8) (width 0.8) (layer "B.Cu") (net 10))
 (segment (start 185.2 105.8) (end 185.2 87) (width 0.8) (layer "B.Cu") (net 10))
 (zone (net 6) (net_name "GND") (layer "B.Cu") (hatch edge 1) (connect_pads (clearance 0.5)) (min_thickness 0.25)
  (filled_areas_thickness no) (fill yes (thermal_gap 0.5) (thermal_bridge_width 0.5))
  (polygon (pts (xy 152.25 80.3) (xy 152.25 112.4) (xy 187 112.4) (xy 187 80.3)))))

